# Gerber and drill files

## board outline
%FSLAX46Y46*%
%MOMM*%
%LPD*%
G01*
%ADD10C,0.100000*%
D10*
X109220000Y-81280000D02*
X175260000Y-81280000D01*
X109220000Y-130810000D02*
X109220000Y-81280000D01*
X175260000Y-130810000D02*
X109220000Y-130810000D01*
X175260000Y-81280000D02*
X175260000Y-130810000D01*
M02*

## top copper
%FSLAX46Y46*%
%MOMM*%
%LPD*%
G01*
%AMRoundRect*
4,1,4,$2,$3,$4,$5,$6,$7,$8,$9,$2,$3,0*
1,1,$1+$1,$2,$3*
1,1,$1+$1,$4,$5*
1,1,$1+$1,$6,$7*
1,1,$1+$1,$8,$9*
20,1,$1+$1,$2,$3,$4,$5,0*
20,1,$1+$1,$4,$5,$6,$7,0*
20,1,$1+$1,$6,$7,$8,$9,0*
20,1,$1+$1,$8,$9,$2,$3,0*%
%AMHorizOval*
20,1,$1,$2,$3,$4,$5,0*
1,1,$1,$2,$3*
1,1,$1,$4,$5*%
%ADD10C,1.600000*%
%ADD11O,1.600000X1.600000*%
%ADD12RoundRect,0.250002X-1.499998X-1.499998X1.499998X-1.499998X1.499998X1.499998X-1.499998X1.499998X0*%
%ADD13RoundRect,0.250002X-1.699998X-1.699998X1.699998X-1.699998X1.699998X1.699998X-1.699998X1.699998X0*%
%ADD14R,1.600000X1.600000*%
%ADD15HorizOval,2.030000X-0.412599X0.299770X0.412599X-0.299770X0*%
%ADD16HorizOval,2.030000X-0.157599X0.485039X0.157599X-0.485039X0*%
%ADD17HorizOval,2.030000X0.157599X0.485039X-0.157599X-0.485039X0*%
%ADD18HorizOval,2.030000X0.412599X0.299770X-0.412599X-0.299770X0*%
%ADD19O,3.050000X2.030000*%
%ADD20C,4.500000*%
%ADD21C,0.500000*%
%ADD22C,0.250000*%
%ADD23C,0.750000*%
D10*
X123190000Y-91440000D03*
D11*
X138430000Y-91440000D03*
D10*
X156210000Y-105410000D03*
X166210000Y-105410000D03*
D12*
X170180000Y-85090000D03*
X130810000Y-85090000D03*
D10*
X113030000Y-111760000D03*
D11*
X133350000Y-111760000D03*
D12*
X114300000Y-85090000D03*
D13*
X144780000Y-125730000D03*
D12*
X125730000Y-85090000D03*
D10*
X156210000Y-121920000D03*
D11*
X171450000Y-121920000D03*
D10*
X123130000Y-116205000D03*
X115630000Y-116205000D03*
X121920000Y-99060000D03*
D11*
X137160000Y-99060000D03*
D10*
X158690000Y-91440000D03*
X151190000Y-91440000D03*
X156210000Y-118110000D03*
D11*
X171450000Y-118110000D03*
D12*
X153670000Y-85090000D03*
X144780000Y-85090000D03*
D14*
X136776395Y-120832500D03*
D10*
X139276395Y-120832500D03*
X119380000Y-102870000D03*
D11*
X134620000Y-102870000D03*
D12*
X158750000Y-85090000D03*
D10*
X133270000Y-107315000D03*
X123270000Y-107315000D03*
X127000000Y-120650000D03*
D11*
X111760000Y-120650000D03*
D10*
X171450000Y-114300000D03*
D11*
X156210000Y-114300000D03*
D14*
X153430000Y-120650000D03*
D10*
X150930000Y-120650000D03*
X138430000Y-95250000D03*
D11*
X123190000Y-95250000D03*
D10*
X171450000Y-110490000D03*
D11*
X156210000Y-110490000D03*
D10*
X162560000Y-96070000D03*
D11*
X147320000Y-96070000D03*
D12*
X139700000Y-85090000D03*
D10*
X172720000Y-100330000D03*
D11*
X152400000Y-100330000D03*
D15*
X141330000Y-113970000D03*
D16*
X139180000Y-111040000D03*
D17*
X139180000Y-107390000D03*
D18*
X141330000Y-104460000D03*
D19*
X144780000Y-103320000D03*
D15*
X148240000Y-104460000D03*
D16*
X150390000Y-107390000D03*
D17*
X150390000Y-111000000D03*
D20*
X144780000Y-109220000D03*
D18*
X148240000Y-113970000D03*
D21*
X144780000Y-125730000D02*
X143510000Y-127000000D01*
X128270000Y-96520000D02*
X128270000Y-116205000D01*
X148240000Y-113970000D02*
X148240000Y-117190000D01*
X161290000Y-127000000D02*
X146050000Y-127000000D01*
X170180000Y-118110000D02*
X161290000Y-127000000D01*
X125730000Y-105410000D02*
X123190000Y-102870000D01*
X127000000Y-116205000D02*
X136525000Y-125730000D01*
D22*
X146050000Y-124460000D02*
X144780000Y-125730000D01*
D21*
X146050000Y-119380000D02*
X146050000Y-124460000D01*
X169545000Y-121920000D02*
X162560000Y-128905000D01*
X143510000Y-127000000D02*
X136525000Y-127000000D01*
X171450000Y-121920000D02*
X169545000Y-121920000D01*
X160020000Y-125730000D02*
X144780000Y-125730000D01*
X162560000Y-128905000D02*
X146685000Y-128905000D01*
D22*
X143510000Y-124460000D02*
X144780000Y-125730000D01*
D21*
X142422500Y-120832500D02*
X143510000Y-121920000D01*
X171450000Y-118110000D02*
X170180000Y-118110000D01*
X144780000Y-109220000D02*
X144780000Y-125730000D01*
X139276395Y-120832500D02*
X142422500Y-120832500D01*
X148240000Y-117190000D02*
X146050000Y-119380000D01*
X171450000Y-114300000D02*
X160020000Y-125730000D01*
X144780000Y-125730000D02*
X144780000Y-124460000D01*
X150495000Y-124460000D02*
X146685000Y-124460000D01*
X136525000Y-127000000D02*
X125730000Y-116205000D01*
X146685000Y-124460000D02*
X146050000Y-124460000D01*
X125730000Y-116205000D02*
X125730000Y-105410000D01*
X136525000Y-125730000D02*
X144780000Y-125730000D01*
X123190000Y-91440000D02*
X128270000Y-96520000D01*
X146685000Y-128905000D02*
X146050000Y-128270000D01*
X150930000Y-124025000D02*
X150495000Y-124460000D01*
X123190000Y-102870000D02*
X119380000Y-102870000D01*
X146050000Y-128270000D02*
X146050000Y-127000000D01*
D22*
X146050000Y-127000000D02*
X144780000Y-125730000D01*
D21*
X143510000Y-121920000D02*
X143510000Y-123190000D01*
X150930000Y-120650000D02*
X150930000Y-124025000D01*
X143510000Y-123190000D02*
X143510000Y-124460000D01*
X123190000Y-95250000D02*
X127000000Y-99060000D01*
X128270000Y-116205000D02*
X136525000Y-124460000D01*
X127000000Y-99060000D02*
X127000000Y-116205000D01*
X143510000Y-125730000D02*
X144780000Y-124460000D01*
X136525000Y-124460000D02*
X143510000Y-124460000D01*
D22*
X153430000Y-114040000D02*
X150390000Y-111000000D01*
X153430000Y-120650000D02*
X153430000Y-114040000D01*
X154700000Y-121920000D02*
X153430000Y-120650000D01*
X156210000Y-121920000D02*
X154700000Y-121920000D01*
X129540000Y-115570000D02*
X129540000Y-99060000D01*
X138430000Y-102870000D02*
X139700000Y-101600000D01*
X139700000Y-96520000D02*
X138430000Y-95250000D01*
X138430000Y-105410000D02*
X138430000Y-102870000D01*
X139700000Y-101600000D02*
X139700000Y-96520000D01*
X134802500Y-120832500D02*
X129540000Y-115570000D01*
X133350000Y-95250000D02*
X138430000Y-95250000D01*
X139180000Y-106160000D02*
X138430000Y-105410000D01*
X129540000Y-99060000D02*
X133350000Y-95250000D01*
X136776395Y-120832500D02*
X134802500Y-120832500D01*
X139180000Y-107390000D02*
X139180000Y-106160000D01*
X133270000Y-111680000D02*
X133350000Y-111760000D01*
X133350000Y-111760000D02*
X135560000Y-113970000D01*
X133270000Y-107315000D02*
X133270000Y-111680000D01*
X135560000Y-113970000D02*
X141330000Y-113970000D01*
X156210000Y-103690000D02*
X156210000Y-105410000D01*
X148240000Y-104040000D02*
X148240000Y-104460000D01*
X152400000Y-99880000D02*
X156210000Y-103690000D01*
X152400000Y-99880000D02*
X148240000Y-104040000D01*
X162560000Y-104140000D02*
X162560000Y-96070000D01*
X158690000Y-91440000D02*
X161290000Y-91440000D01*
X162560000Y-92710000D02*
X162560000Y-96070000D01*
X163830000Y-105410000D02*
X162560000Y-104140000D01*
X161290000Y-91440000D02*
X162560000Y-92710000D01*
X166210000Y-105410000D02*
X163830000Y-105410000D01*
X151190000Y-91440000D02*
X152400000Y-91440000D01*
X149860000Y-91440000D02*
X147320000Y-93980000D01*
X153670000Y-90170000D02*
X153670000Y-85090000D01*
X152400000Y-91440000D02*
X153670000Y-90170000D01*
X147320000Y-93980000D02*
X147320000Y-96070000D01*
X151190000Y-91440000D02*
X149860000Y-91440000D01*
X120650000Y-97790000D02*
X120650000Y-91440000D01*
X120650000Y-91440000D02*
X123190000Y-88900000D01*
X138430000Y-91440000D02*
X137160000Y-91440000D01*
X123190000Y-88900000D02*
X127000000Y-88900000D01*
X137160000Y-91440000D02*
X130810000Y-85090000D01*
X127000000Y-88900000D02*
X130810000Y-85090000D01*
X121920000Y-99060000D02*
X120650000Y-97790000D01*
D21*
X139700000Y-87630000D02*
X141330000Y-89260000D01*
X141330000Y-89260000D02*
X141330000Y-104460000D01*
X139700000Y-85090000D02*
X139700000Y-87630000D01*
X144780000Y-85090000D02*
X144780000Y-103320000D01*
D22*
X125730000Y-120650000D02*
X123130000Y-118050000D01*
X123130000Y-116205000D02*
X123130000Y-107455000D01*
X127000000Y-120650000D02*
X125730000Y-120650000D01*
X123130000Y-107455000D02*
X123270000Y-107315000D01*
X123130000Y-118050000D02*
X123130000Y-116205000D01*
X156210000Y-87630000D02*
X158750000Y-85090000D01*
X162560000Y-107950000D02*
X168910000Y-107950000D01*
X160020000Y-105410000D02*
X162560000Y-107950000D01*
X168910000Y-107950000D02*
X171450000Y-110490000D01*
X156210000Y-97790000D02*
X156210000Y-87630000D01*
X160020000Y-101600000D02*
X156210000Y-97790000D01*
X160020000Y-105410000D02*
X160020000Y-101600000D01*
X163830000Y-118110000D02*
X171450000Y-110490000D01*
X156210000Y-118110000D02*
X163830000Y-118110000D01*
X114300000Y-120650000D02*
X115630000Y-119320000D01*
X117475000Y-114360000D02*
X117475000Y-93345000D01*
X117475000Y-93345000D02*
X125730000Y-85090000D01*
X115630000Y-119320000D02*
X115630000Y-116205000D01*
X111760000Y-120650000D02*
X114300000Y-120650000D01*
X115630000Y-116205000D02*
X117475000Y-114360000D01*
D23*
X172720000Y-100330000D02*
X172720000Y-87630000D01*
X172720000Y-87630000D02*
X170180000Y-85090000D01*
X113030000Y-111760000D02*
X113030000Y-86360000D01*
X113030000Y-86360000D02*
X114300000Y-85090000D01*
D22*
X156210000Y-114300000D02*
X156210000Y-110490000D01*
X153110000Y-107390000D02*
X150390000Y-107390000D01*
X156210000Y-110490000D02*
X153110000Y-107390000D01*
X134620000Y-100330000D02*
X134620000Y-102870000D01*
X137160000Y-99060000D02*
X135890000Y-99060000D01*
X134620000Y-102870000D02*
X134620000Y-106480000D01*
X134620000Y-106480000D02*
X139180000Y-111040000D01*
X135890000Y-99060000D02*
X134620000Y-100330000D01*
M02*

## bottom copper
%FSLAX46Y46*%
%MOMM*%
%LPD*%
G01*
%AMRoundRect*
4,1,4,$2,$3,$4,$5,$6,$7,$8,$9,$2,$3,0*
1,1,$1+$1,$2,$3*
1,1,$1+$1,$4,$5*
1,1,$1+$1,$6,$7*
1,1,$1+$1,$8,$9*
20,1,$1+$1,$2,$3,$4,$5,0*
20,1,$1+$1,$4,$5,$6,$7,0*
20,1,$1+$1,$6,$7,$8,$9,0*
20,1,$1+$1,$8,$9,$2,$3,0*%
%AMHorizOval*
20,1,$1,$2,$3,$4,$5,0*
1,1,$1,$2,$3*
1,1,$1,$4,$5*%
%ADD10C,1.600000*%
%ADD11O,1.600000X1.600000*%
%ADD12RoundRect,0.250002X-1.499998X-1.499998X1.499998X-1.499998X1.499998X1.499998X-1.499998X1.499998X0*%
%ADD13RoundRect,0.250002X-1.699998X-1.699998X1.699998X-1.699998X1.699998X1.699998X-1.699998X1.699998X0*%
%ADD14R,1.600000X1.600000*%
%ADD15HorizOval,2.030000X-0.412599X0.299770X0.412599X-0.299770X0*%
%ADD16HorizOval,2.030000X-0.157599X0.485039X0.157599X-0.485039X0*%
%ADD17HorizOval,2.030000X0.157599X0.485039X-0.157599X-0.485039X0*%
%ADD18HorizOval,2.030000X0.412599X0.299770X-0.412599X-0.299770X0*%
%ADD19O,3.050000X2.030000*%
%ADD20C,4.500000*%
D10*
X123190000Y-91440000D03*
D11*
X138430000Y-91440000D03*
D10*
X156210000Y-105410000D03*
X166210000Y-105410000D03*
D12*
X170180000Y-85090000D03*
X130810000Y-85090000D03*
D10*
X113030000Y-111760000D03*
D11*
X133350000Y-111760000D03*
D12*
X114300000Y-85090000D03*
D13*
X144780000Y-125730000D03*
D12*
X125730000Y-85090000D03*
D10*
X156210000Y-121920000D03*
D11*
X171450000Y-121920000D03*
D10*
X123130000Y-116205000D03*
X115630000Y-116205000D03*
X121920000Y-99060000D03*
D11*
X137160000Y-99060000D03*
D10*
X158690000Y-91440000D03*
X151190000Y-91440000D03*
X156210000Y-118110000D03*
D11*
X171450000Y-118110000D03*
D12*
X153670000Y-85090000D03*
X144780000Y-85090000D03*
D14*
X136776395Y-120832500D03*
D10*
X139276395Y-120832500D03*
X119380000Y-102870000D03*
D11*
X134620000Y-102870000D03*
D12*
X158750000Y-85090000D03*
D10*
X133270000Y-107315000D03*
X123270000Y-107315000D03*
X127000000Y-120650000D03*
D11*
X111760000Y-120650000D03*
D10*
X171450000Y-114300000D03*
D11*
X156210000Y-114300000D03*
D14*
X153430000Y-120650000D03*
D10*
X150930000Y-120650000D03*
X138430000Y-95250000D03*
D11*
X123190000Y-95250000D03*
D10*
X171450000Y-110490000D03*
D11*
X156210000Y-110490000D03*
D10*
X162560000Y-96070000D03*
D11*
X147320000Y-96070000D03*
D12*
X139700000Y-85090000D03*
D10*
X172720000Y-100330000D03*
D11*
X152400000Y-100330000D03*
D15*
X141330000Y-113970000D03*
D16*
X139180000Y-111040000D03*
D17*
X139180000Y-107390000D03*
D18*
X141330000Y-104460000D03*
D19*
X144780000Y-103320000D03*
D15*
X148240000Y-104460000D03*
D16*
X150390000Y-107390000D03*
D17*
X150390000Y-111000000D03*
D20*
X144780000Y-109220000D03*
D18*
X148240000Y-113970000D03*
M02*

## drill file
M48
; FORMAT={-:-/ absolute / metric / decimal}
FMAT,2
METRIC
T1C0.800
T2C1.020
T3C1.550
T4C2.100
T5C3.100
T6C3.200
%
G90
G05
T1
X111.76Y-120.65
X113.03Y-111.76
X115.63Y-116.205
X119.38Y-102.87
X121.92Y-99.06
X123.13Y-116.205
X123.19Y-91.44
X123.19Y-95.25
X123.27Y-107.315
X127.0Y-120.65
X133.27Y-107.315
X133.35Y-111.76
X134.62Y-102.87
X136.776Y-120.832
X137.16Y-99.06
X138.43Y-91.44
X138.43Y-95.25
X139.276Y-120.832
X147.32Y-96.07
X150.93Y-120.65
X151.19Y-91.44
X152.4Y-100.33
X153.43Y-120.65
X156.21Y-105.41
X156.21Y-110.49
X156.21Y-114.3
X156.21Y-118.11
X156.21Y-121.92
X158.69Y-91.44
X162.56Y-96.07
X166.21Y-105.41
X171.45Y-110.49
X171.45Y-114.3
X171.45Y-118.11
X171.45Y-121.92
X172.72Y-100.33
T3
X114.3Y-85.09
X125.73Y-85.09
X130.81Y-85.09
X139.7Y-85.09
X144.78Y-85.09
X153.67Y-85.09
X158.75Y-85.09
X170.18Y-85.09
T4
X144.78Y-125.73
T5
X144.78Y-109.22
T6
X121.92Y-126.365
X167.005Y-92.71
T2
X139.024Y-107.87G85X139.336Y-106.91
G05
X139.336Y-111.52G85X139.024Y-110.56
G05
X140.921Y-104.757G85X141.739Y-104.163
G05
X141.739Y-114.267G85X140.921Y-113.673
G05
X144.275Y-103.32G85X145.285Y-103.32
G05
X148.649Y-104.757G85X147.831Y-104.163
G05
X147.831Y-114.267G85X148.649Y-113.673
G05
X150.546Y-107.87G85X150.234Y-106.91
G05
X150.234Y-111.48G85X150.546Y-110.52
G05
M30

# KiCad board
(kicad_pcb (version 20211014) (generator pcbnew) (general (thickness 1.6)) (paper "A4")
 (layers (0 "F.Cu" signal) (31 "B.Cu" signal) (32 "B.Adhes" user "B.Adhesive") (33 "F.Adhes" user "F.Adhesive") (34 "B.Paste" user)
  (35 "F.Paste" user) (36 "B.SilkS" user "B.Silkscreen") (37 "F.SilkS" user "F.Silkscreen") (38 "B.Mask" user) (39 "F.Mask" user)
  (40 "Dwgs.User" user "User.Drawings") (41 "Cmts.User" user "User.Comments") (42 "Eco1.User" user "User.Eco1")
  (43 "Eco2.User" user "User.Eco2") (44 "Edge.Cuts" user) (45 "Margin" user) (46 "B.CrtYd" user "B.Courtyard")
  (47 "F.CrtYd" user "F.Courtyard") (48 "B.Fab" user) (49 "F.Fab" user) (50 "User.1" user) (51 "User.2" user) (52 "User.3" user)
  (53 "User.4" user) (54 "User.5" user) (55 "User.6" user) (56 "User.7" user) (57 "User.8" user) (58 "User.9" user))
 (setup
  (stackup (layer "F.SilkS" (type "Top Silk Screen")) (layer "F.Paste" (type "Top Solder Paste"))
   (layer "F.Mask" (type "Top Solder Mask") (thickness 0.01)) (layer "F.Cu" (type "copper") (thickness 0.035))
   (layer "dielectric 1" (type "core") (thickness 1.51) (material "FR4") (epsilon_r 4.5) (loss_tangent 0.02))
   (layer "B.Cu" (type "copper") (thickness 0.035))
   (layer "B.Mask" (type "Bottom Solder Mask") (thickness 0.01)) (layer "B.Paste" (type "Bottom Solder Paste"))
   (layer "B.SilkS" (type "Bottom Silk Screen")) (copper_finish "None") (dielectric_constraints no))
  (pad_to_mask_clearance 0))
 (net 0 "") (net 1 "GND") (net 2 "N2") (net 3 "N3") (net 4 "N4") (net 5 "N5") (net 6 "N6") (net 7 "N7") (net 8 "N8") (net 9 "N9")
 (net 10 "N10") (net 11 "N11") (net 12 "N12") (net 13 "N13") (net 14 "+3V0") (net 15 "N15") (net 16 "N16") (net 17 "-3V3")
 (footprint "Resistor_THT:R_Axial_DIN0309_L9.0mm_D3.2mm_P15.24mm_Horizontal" (layer "F.Cu") (at 123.19 91.44)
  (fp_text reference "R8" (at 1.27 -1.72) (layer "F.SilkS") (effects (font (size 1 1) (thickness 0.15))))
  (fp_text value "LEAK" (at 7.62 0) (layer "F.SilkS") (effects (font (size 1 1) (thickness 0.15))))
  (pad "1" thru_hole circle (at 0 0) (size 1.6 1.6) (drill 0.8) (layers *.Cu *.Mask) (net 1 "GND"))
  (pad "2" thru_hole oval (at 15.24 0) (size 1.6 1.6) (drill 0.8) (layers *.Cu *.Mask) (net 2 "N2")))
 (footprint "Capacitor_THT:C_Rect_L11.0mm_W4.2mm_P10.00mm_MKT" (layer "F.Cu") (at 156.21 105.41)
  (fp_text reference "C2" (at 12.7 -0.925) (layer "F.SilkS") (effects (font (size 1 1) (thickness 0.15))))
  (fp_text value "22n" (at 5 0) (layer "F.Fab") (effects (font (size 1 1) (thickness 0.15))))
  (pad "1" thru_hole circle (at 0 0) (size 1.6 1.6) (drill 0.8) (layers *.Cu *.Mask) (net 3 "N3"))
  (pad "2" thru_hole circle (at 10 0) (size 1.6 1.6) (drill 0.8) (layers *.Cu *.Mask) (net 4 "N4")))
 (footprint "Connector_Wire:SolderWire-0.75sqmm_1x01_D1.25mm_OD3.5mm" (layer "F.Cu") (at 170.18 85.09)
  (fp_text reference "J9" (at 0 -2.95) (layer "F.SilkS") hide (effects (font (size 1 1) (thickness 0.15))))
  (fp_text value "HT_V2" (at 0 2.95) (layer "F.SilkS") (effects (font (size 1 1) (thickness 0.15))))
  (pad "1" thru_hole roundrect (at 0 0) (size 3.5 3.5) (drill 1.55) (layers *.Cu *.Mask) (roundrect_rratio 0.07142914286) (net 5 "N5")))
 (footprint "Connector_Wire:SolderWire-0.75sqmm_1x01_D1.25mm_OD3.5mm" (layer "F.Cu") (at 130.81 85.09)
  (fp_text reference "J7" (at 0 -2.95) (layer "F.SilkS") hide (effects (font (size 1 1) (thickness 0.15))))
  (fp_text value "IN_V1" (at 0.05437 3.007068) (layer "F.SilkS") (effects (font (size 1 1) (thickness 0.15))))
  (pad "1" thru_hole roundrect (at 0 0) (size 3.5 3.5) (drill 1.55) (layers *.Cu *.Mask) (roundrect_rratio 0.07142914286) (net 2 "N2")))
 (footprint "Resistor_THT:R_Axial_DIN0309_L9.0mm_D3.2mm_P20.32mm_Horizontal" (layer "F.Cu") (at 113.03 111.76)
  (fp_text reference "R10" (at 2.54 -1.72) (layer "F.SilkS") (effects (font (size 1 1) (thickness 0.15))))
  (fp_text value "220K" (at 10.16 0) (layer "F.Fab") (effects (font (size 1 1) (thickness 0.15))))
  (pad "1" thru_hole circle (at 0 0) (size 1.6 1.6) (drill 0.8) (layers *.Cu *.Mask) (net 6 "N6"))
  (pad "2" thru_hole oval (at 20.32 0) (size 1.6 1.6) (drill 0.8) (layers *.Cu *.Mask) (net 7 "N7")))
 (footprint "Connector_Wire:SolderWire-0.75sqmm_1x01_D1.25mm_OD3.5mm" (layer "F.Cu") (at 114.3 85.09)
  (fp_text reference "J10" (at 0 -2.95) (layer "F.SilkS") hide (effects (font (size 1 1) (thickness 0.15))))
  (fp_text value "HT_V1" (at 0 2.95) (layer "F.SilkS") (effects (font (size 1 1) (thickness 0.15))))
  (pad "1" thru_hole roundrect (at 0 0) (size 3.5 3.5) (drill 1.55) (layers *.Cu *.Mask) (roundrect_rratio 0.07142914286) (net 6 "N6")))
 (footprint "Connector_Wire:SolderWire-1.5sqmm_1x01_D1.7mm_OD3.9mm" (layer "F.Cu") (at 144.78 125.73)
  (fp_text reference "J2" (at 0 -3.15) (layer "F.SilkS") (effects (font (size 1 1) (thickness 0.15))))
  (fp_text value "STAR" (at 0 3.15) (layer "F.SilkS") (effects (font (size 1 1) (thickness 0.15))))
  (pad "1" thru_hole roundrect (at 0 0) (size 3.9 3.9) (drill 2.1) (layers *.Cu *.Mask) (roundrect_rratio 0.06410307692) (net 1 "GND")))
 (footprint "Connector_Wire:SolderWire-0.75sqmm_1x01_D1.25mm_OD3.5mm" (layer "F.Cu") (at 125.73 85.09)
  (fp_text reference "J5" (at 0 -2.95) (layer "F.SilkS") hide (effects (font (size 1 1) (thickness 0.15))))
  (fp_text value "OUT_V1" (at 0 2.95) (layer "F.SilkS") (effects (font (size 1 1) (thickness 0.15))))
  (pad "1" thru_hole roundrect (at 0 0) (size 3.5 3.5) (drill 1.55) (layers *.Cu *.Mask) (roundrect_rratio 0.07142914286) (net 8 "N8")))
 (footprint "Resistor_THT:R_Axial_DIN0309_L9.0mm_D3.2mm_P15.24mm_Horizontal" (layer "F.Cu") (at 156.21 121.92)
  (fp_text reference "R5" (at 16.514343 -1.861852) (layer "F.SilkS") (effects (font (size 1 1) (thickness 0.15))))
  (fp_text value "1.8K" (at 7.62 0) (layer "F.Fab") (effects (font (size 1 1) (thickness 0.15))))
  (pad "1" thru_hole circle (at 0 0) (size 1.6 1.6) (drill 0.8) (layers *.Cu *.Mask) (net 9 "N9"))
  (pad "2" thru_hole oval (at 15.24 0) (size 1.6 1.6) (drill 0.8) (layers *.Cu *.Mask) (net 1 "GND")))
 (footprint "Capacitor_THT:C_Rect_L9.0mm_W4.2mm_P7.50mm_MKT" (layer "F.Cu") (at 123.13 116.205 180)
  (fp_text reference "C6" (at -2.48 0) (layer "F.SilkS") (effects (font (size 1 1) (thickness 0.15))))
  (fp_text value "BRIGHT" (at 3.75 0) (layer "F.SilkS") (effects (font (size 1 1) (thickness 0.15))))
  (pad "1" thru_hole circle (at 0 0 180) (size 1.6 1.6) (drill 0.8) (layers *.Cu *.Mask) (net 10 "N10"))
  (pad "2" thru_hole circle (at 7.5 0 180) (size 1.6 1.6) (drill 0.8) (layers *.Cu *.Mask) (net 8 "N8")))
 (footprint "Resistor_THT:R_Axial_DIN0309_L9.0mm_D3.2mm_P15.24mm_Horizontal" (layer "F.Cu") (at 121.92 99.06)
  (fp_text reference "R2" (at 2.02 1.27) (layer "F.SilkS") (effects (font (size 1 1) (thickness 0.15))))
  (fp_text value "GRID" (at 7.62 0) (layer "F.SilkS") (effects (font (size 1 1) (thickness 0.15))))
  (pad "1" thru_hole circle (at 0 0) (size 1.6 1.6) (drill 0.8) (layers *.Cu *.Mask) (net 2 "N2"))
  (pad "2" thru_hole oval (at 15.24 0) (size 1.6 1.6) (drill 0.8) (layers *.Cu *.Mask) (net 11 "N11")))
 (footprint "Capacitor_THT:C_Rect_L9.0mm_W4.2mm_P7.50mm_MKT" (layer "F.Cu") (at 158.69 91.44 180)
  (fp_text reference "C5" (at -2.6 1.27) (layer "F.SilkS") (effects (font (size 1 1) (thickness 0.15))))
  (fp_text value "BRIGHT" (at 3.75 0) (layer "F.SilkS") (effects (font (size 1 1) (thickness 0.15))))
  (pad "1" thru_hole circle (at 0 0 180) (size 1.6 1.6) (drill 0.8) (layers *.Cu *.Mask) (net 4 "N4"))
  (pad "2" thru_hole circle (at 7.5 0 180) (size 1.6 1.6) (drill 0.8) (layers *.Cu *.Mask) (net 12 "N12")))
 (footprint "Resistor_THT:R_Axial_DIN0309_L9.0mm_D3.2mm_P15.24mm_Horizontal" (layer "F.Cu") (at 156.21 118.11)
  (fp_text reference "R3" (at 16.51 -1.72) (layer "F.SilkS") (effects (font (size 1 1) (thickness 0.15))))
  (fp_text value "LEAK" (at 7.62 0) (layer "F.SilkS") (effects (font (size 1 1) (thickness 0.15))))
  (pad "1" thru_hole circle (at 0 0) (size 1.6 1.6) (drill 0.8) (layers *.Cu *.Mask) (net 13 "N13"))
  (pad "2" thru_hole oval (at 15.24 0) (size 1.6 1.6) (drill 0.8) (layers *.Cu *.Mask) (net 1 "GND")))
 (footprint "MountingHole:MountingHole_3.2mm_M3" (layer "F.Cu") (at 167.005 92.71)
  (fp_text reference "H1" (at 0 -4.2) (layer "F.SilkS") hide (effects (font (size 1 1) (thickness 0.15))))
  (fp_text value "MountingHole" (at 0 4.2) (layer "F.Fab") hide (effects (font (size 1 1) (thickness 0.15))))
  (pad "" np_thru_hole circle (at 0 0) (size 3.2 3.2) (drill 3.2) (layers *.Cu *.Mask)))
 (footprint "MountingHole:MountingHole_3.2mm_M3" (layer "F.Cu") (at 121.92 126.365)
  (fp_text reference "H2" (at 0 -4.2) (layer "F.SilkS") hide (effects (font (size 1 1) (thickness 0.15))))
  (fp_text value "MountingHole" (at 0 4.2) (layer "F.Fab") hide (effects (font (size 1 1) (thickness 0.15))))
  (pad "" np_thru_hole circle (at 0 0) (size 3.2 3.2) (drill 3.2) (layers *.Cu *.Mask)))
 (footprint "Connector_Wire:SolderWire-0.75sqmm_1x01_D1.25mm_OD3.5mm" (layer "F.Cu") (at 153.67 85.09)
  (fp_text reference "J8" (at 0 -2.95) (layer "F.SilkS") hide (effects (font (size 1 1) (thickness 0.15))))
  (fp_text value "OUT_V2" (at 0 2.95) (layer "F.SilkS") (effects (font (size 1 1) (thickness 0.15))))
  (pad "1" thru_hole roundrect (at 0 0) (size 3.5 3.5) (drill 1.55) (layers *.Cu *.Mask) (roundrect_rratio 0.07142914286) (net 12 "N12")))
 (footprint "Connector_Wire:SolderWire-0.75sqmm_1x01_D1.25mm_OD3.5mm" (layer "F.Cu") (at 144.78 85.09)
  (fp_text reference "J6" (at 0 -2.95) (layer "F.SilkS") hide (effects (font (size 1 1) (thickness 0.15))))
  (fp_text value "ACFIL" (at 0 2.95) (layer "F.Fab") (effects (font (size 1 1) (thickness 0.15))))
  (pad "1" thru_hole roundrect (at 0 0) (size 3.5 3.5) (drill 1.55) (layers *.Cu *.Mask) (roundrect_rratio 0.07142914286) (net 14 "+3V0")))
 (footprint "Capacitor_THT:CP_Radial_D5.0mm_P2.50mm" (layer "F.Cu") (at 136.776395 120.8325)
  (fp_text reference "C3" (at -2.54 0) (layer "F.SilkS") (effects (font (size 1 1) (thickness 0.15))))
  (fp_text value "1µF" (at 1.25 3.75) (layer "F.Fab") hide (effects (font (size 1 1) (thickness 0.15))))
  (pad "1" thru_hole rect (at 0 0) (size 1.6 1.6) (drill 0.8) (layers *.Cu *.Mask) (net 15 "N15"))
  (pad "2" thru_hole circle (at 2.5 0) (size 1.6 1.6) (drill 0.8) (layers *.Cu *.Mask) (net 1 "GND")))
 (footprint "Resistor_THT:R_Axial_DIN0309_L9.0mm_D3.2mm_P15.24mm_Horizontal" (layer "F.Cu") (at 119.38 102.87)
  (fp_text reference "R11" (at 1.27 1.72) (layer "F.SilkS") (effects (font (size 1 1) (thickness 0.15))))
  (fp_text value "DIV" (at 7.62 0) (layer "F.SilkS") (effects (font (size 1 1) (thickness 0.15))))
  (pad "1" thru_hole circle (at 0 0) (size 1.6 1.6) (drill 0.8) (layers *.Cu *.Mask) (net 1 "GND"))
  (pad "2" thru_hole oval (at 15.24 0) (size 1.6 1.6) (drill 0.8) (layers *.Cu *.Mask) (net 11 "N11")))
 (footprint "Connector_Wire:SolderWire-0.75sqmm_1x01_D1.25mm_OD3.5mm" (layer "F.Cu") (at 158.75 85.09)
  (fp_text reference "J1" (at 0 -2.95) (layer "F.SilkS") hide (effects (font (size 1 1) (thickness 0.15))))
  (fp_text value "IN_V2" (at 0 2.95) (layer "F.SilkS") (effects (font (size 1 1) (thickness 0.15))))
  (pad "1" thru_hole roundrect (at 0 0) (size 3.5 3.5) (drill 1.55) (layers *.Cu *.Mask) (roundrect_rratio 0.07142914286) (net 13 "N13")))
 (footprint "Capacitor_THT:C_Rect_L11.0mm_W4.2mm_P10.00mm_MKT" (layer "F.Cu") (at 133.27 107.315 180)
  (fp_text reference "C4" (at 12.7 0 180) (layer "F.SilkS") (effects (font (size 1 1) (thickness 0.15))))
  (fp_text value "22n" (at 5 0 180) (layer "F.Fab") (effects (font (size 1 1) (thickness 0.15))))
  (pad "1" thru_hole circle (at 0 0 180) (size 1.6 1.6) (drill 0.8) (layers *.Cu *.Mask) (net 7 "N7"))
  (pad "2" thru_hole circle (at 10 0 180) (size 1.6 1.6) (drill 0.8) (layers *.Cu *.Mask) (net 10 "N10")))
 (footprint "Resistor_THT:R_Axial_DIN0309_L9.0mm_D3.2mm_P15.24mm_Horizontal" (layer "F.Cu") (at 127 120.65 180)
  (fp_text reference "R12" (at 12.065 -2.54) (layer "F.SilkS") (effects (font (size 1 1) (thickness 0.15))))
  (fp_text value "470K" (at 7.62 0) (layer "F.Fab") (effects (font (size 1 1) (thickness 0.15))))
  (pad "1" thru_hole circle (at 0 0 180) (size 1.6 1.6) (drill 0.8) (layers *.Cu *.Mask) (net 10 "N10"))
  (pad "2" thru_hole oval (at 15.24 0 180) (size 1.6 1.6) (drill 0.8) (layers *.Cu *.Mask) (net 8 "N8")))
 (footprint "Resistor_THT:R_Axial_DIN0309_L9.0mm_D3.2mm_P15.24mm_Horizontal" (layer "F.Cu") (at 171.45 114.3 180)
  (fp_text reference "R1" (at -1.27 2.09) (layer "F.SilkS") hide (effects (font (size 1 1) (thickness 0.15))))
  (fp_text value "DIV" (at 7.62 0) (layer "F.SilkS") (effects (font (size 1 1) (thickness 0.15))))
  (pad "1" thru_hole circle (at 0 0 180) (size 1.6 1.6) (drill 0.8) (layers *.Cu *.Mask) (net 1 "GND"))
  (pad "2" thru_hole oval (at 15.24 0 180) (size 1.6 1.6) (drill 0.8) (layers *.Cu *.Mask) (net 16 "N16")))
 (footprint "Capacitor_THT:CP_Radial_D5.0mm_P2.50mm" (layer "F.Cu") (at 153.43 120.65 180)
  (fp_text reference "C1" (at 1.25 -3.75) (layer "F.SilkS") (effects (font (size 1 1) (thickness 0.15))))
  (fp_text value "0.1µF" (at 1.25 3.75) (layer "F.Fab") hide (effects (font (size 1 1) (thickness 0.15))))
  (pad "1" thru_hole rect (at 0 0 180) (size 1.6 1.6) (drill 0.8) (layers *.Cu *.Mask) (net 9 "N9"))
  (pad "2" thru_hole circle (at 2.5 0 180) (size 1.6 1.6) (drill 0.8) (layers *.Cu *.Mask) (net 1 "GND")))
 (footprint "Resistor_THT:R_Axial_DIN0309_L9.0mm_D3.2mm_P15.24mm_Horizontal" (layer "F.Cu") (at 138.43 95.25 180)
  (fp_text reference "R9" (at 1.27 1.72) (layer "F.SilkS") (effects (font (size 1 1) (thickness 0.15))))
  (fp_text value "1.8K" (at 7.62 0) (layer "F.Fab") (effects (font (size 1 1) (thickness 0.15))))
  (pad "1" thru_hole circle (at 0 0 180) (size 1.6 1.6) (drill 0.8) (layers *.Cu *.Mask) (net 15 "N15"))
  (pad "2" thru_hole oval (at 15.24 0 180) (size 1.6 1.6) (drill 0.8) (layers *.Cu *.Mask) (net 1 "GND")))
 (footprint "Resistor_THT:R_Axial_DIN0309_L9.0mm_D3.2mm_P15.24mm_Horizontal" (layer "F.Cu") (at 171.45 110.49 180)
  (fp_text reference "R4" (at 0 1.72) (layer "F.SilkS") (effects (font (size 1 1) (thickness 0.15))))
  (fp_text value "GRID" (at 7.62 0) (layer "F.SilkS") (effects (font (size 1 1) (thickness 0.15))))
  (pad "1" thru_hole circle (at 0 0 180) (size 1.6 1.6) (drill 0.8) (layers *.Cu *.Mask) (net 13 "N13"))
  (pad "2" thru_hole oval (at 15.24 0 180) (size 1.6 1.6) (drill 0.8) (layers *.Cu *.Mask) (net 16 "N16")))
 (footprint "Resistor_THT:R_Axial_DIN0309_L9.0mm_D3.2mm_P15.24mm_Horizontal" (layer "F.Cu") (at 162.56 96.07 180)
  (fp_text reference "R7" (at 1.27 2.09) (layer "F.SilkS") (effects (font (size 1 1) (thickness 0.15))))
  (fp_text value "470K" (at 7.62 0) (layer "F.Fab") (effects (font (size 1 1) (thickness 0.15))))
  (pad "1" thru_hole circle (at 0 0 180) (size 1.6 1.6) (drill 0.8) (layers *.Cu *.Mask) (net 4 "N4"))
  (pad "2" thru_hole oval (at 15.24 0 180) (size 1.6 1.6) (drill 0.8) (layers *.Cu *.Mask) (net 12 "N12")))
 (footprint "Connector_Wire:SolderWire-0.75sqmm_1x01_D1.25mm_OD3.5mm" (layer "F.Cu") (at 139.7 85.09)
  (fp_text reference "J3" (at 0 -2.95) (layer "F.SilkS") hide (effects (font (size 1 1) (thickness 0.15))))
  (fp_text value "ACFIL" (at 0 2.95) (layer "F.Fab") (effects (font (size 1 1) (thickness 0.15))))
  (pad "1" thru_hole roundrect (at 0 0) (size 3.5 3.5) (drill 1.55) (layers *.Cu *.Mask) (roundrect_rratio 0.07142914286) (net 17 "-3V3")))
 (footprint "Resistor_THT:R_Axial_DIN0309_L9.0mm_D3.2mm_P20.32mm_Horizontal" (layer "F.Cu") (at 172.72 100.33 180)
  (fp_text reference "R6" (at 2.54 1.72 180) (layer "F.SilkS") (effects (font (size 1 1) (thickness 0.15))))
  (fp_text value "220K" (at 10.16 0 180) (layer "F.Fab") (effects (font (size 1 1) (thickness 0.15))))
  (pad "1" thru_hole circle (at 0 0 180) (size 1.6 1.6) (drill 0.8) (layers *.Cu *.Mask) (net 5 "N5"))
  (pad "2" thru_hole oval (at 20.32 0 180) (size 1.6 1.6) (drill 0.8) (layers *.Cu *.Mask) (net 3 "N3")))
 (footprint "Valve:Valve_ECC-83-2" (layer "B.Cu") (at 141.33 113.97 180)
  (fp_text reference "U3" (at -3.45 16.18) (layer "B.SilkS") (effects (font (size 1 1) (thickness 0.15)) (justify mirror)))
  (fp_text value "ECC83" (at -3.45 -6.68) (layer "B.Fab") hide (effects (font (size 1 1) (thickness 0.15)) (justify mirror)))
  (pad "1" thru_hole oval (at 0 0 234) (size 2.03 3.05) (drill oval 1.02 2.03) (layers *.Cu *.Mask) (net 7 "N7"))
  (pad "2" thru_hole oval (at 2.15 2.93 198) (size 2.03 3.05) (drill oval 1.02 2.03) (layers *.Cu *.Mask) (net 11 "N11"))
  (pad "3" thru_hole oval (at 2.15 6.58 162) (size 2.03 3.05) (drill oval 1.02 2.03) (layers *.Cu *.Mask) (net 15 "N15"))
  (pad "4" thru_hole oval (at 0 9.51 126) (size 2.03 3.05) (drill oval 1.02 2.03) (layers *.Cu *.Mask) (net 17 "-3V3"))
  (pad "5" thru_hole oval (at -3.45 10.65 90) (size 2.03 3.05) (drill oval 1.02 2.03) (layers *.Cu *.Mask) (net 14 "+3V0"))
  (pad "6" thru_hole oval (at -6.91 9.51 234) (size 2.03 3.05) (drill oval 1.02 2.03) (layers *.Cu *.Mask) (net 3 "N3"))
  (pad "7" thru_hole oval (at -9.06 6.58 198) (size 2.03 3.05) (drill oval 1.02 2.03) (layers *.Cu *.Mask) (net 16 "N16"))
  (pad "8" thru_hole oval (at -9.06 2.97 162) (size 2.03 3.05) (drill oval 1.02 2.03) (layers *.Cu *.Mask) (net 9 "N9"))
  (pad "9" thru_hole circle (at -3.45 4.75 180) (size 4.5 4.5) (drill 3.1) (layers *.Cu *.Mask) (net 1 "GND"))
  (pad "9" thru_hole oval (at -6.91 0 126) (size 2.03 3.05) (drill oval 1.02 2.03) (layers *.Cu *.Mask) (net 1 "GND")))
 (gr_line (start 109.22 81.28) (end 175.26 81.28) (layer "Edge.Cuts") (width 0.1))
 (gr_line (start 109.22 130.81) (end 109.22 81.28) (layer "Edge.Cuts") (width 0.1))
 (gr_line (start 175.26 130.81) (end 109.22 130.81) (layer "Edge.Cuts") (width 0.1))
 (gr_line (start 175.26 81.28) (end 175.26 130.81) (layer "Edge.Cuts") (width 0.1))
 (segment (start 144.78 125.73) (end 143.51 127) (width 0.5) (layer "F.Cu") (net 1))
 (segment (start 128.27 96.52) (end 128.27 116.205) (width 0.5) (layer "F.Cu") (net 1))
 (segment (start 148.24 113.97) (end 148.24 117.19) (width 0.5) (layer "F.Cu") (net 1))
 (segment (start 161.29 127) (end 146.05 127) (width 0.5) (layer "F.Cu") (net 1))
 (segment (start 170.18 118.11) (end 161.29 127) (width 0.5) (layer "F.Cu") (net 1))
 (segment (start 125.73 105.41) (end 123.19 102.87) (width 0.5) (layer "F.Cu") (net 1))
 (segment (start 127 116.205) (end 136.525 125.73) (width 0.5) (layer "F.Cu") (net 1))
 (segment (start 146.05 124.46) (end 144.78 125.73) (width 0.25) (layer "F.Cu") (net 1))
 (segment (start 146.05 119.38) (end 146.05 124.46) (width 0.5) (layer "F.Cu") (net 1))
 (segment (start 169.545 121.92) (end 162.56 128.905) (width 0.5) (layer "F.Cu") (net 1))
 (segment (start 143.51 127) (end 136.525 127) (width 0.5) (layer "F.Cu") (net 1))
 (segment (start 171.45 121.92) (end 169.545 121.92) (width 0.5) (layer "F.Cu") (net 1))
 (segment (start 160.02 125.73) (end 144.78 125.73) (width 0.5) (layer "F.Cu") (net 1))
 (segment (start 162.56 128.905) (end 146.685 128.905) (width 0.5) (layer "F.Cu") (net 1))
 (segment (start 143.51 124.46) (end 144.78 125.73) (width 0.25) (layer "F.Cu") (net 1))
 (segment (start 142.4225 120.8325) (end 143.51 121.92) (width 0.5) (layer "F.Cu") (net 1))
 (segment (start 171.45 118.11) (end 170.18 118.11) (width 0.5) (layer "F.Cu") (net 1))
 (segment (start 144.78 109.22) (end 144.78 125.73) (width 0.5) (layer "F.Cu") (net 1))
 (segment (start 139.276395 120.8325) (end 142.4225 120.8325) (width 0.5) (layer "F.Cu") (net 1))
 (segment (start 148.24 117.19) (end 146.05 119.38) (width 0.5) (layer "F.Cu") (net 1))
 (segment (start 171.45 114.3) (end 160.02 125.73) (width 0.5) (layer "F.Cu") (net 1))
 (segment (start 144.78 125.73) (end 144.78 124.46) (width 0.5) (layer "F.Cu") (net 1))
 (segment (start 150.495 124.46) (end 146.685 124.46) (width 0.5) (layer "F.Cu") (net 1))
 (segment (start 136.525 127) (end 125.73 116.205) (width 0.5) (layer "F.Cu") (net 1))
 (segment (start 146.685 124.46) (end 146.05 124.46) (width 0.5) (layer "F.Cu") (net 1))
 (segment (start 125.73 116.205) (end 125.73 105.41) (width 0.5) (layer "F.Cu") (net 1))
 (segment (start 136.525 125.73) (end 144.78 125.73) (width 0.5) (layer "F.Cu") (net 1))
 (segment (start 123.19 91.44) (end 128.27 96.52) (width 0.5) (layer "F.Cu") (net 1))
 (segment (start 146.685 128.905) (end 146.05 128.27) (width 0.5) (layer "F.Cu") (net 1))
 (segment (start 150.93 124.025) (end 150.495 124.46) (width 0.5) (layer "F.Cu") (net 1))
 (segment (start 123.19 102.87) (end 119.38 102.87) (width 0.5) (layer "F.Cu") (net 1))
 (segment (start 146.05 128.27) (end 146.05 127) (width 0.5) (layer "F.Cu") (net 1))
 (segment (start 146.05 127) (end 144.78 125.73) (width 0.25) (layer "F.Cu") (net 1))
 (segment (start 143.51 121.92) (end 143.51 123.19) (width 0.5) (layer "F.Cu") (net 1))
 (segment (start 150.93 120.65) (end 150.93 124.025) (width 0.5) (layer "F.Cu") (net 1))
 (segment (start 143.51 123.19) (end 143.51 124.46) (width 0.5) (layer "F.Cu") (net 1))
 (segment (start 123.19 95.25) (end 127 99.06) (width 0.5) (layer "F.Cu") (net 1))
 (segment (start 128.27 116.205) (end 136.525 124.46) (width 0.5) (layer "F.Cu") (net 1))
 (segment (start 127 99.06) (end 127 116.205) (width 0.5) (layer "F.Cu") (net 1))
 (segment (start 143.51 125.73) (end 144.78 124.46) (width 0.5) (layer "F.Cu") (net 1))
 (segment (start 136.525 124.46) (end 143.51 124.46) (width 0.5) (layer "F.Cu") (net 1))
 (segment (start 153.43 114.04) (end 150.39 111) (width 0.25) (layer "F.Cu") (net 9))
 (segment (start 153.43 120.65) (end 153.43 114.04) (width 0.25) (layer "F.Cu") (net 9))
 (segment (start 154.7 121.92) (end 153.43 120.65) (width 0.25) (layer "F.Cu") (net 9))
 (segment (start 156.21 121.92) (end 154.7 121.92) (width 0.25) (layer "F.Cu") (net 9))
 (segment (start 129.54 115.57) (end 129.54 99.06) (width 0.25) (layer "F.Cu") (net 15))
 (segment (start 138.43 102.87) (end 139.7 101.6) (width 0.25) (layer "F.Cu") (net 15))
 (segment (start 139.7 96.52) (end 138.43 95.25) (width 0.25) (layer "F.Cu") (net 15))
 (segment (start 138.43 105.41) (end 138.43 102.87) (width 0.25) (layer "F.Cu") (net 15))
 (segment (start 139.7 101.6) (end 139.7 96.52) (width 0.25) (layer "F.Cu") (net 15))
 (segment (start 134.8025 120.8325) (end 129.54 115.57) (width 0.25) (layer "F.Cu") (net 15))
 (segment (start 133.35 95.25) (end 138.43 95.25) (width 0.25) (layer "F.Cu") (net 15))
 (segment (start 139.18 106.16) (end 138.43 105.41) (width 0.25) (layer "F.Cu") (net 15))
 (segment (start 129.54 99.06) (end 133.35 95.25) (width 0.25) (layer "F.Cu") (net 15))
 (segment (start 136.776395 120.8325) (end 134.8025 120.8325) (width 0.25) (layer "F.Cu") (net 15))
 (segment (start 139.18 107.39) (end 139.18 106.16) (width 0.25) (layer "F.Cu") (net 15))
 (segment (start 133.27 111.68) (end 133.35 111.76) (width 0.25) (layer "F.Cu") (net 7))
 (segment (start 133.35 111.76) (end 135.56 113.97) (width 0.25) (layer "F.Cu") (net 7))
 (segment (start 133.27 107.315) (end 133.27 111.68) (width 0.25) (layer "F.Cu") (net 7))
 (segment (start 135.56 113.97) (end 141.33 113.97) (width 0.25) (layer "F.Cu") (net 7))
 (segment (start 156.21 103.69) (end 156.21 105.41) (width 0.25) (layer "F.Cu") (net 3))
 (segment (start 148.24 104.04) (end 148.24 104.46) (width 0.25) (layer "F.Cu") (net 3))
 (segment (start 152.4 99.88) (end 156.21 103.69) (width 0.25) (layer "F.Cu") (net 3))
 (segment (start 152.4 99.88) (end 148.24 104.04) (width 0.25) (layer "F.Cu") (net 3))
 (segment (start 162.56 104.14) (end 162.56 96.07) (width 0.25) (layer "F.Cu") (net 4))
 (segment (start 158.69 91.44) (end 161.29 91.44) (width 0.25) (layer "F.Cu") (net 4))
 (segment (start 162.56 92.71) (end 162.56 96.07) (width 0.25) (layer "F.Cu") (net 4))
 (segment (start 163.83 105.41) (end 162.56 104.14) (width 0.25) (layer "F.Cu") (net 4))
 (segment (start 161.29 91.44) (end 162.56 92.71) (width 0.25) (layer "F.Cu") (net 4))
 (segment (start 166.21 105.41) (end 163.83 105.41) (width 0.25) (layer "F.Cu") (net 4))
 (segment (start 151.19 91.44) (end 152.4 91.44) (width 0.25) (layer "F.Cu") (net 12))
 (segment (start 149.86 91.44) (end 147.32 93.98) (width 0.25) (layer "F.Cu") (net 12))
 (segment (start 153.67 90.17) (end 153.67 85.09) (width 0.25) (layer "F.Cu") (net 12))
 (segment (start 152.4 91.44) (end 153.67 90.17) (width 0.25) (layer "F.Cu") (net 12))
 (segment (start 147.32 93.98) (end 147.32 96.07) (width 0.25) (layer "F.Cu") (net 12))
 (segment (start 151.19 91.44) (end 149.86 91.44) (width 0.25) (layer "F.Cu") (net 12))
 (segment (start 120.65 97.79) (end 120.65 91.44) (width 0.25) (layer "F.Cu") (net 2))
 (segment (start 120.65 91.44) (end 123.19 88.9) (width 0.25) (layer "F.Cu") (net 2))
 (segment (start 138.43 91.44) (end 137.16 91.44) (width 0.25) (layer "F.Cu") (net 2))
 (segment (start 123.19 88.9) (end 127 88.9) (width 0.25) (layer "F.Cu") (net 2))
 (segment (start 137.16 91.44) (end 130.81 85.09) (width 0.25) (layer "F.Cu") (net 2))
 (segment (start 127 88.9) (end 130.81 85.09) (width 0.25) (layer "F.Cu") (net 2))
 (segment (start 121.92 99.06) (end 120.65 97.79) (width 0.25) (layer "F.Cu") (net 2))
 (segment (start 139.7 87.63) (end 141.33 89.26) (width 0.5) (layer "F.Cu") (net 17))
 (segment (start 141.33 89.26) (end 141.33 104.46) (width 0.5) (layer "F.Cu") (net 17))
 (segment (start 139.7 85.09) (end 139.7 87.63) (width 0.5) (layer "F.Cu") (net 17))
 (segment (start 144.78 85.09) (end 144.78 103.32) (width 0.5) (layer "F.Cu") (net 14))
 (segment (start 125.73 120.65) (end 123.13 118.05) (width 0.25) (layer "F.Cu") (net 10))
 (segment (start 123.13 116.205) (end 123.13 107.455) (width 0.25) (layer "F.Cu") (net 10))
 (segment (start 127 120.65) (end 125.73 120.65) (width 0.25) (layer "F.Cu") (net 10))
 (segment (start 123.13 107.455) (end 123.27 107.315) (width 0.25) (layer "F.Cu") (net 10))
 (segment (start 123.13 118.05) (end 123.13 116.205) (width 0.25) (layer "F.Cu") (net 10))
 (segment (start 156.21 87.63) (end 158.75 85.09) (width 0.25) (layer "F.Cu") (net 13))
 (segment (start 162.56 107.95) (end 168.91 107.95) (width 0.25) (layer "F.Cu") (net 13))
 (segment (start 160.02 105.41) (end 162.56 107.95) (width 0.25) (layer "F.Cu") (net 13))
 (segment (start 168.91 107.95) (end 171.45 110.49) (width 0.25) (layer "F.Cu") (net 13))
 (segment (start 156.21 97.79) (end 156.21 87.63) (width 0.25) (layer "F.Cu") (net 13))
 (segment (start 160.02 101.6) (end 156.21 97.79) (width 0.25) (layer "F.Cu") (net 13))
 (segment (start 160.02 105.41) (end 160.02 101.6) (width 0.25) (layer "F.Cu") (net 13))
 (segment (start 163.83 118.11) (end 171.45 110.49) (width 0.25) (layer "F.Cu") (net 13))
 (segment (start 156.21 118.11) (end 163.83 118.11) (width 0.25) (layer "F.Cu") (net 13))
 (segment (start 114.3 120.65) (end 115.63 119.32) (width 0.25) (layer "F.Cu") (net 8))
 (segment (start 117.475 114.36) (end 117.475 93.345) (width 0.25) (layer "F.Cu") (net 8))
 (segment (start 117.475 93.345) (end 125.73 85.09) (width 0.25) (layer "F.Cu") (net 8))
 (segment (start 115.63 119.32) (end 115.63 116.205) (width 0.25) (layer "F.Cu") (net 8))
 (segment (start 111.76 120.65) (end 114.3 120.65) (width 0.25) (layer "F.Cu") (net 8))
 (segment (start 115.63 116.205) (end 117.475 114.36) (width 0.25) (layer "F.Cu") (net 8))
 (segment (start 172.72 100.33) (end 172.72 87.63) (width 0.75) (layer "F.Cu") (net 5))
 (segment (start 172.72 87.63) (end 170.18 85.09) (width 0.75) (layer "F.Cu") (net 5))
 (segment (start 113.03 111.76) (end 113.03 86.36) (width 0.75) (layer "F.Cu") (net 6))
 (segment (start 113.03 86.36) (end 114.3 85.09) (width 0.75) (layer "F.Cu") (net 6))
 (segment (start 156.21 114.3) (end 156.21 110.49) (width 0.25) (layer "F.Cu") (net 16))
 (segment (start 153.11 107.39) (end 150.39 107.39) (width 0.25) (layer "F.Cu") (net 16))
 (segment (start 156.21 110.49) (end 153.11 107.39) (width 0.25) (layer "F.Cu") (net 16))
 (segment (start 134.62 100.33) (end 134.62 102.87) (width 0.25) (layer "F.Cu") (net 11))
 (segment (start 137.16 99.06) (end 135.89 99.06) (width 0.25) (layer "F.Cu") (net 11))
 (segment (start 134.62 102.87) (end 134.62 106.48) (width 0.25) (layer "F.Cu") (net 11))
 (segment (start 134.62 106.48) (end 139.18 111.04) (width 0.25) (layer "F.Cu") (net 11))
 (segment (start 135.89 99.06) (end 134.62 100.33) (width 0.25) (layer "F.Cu") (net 11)))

